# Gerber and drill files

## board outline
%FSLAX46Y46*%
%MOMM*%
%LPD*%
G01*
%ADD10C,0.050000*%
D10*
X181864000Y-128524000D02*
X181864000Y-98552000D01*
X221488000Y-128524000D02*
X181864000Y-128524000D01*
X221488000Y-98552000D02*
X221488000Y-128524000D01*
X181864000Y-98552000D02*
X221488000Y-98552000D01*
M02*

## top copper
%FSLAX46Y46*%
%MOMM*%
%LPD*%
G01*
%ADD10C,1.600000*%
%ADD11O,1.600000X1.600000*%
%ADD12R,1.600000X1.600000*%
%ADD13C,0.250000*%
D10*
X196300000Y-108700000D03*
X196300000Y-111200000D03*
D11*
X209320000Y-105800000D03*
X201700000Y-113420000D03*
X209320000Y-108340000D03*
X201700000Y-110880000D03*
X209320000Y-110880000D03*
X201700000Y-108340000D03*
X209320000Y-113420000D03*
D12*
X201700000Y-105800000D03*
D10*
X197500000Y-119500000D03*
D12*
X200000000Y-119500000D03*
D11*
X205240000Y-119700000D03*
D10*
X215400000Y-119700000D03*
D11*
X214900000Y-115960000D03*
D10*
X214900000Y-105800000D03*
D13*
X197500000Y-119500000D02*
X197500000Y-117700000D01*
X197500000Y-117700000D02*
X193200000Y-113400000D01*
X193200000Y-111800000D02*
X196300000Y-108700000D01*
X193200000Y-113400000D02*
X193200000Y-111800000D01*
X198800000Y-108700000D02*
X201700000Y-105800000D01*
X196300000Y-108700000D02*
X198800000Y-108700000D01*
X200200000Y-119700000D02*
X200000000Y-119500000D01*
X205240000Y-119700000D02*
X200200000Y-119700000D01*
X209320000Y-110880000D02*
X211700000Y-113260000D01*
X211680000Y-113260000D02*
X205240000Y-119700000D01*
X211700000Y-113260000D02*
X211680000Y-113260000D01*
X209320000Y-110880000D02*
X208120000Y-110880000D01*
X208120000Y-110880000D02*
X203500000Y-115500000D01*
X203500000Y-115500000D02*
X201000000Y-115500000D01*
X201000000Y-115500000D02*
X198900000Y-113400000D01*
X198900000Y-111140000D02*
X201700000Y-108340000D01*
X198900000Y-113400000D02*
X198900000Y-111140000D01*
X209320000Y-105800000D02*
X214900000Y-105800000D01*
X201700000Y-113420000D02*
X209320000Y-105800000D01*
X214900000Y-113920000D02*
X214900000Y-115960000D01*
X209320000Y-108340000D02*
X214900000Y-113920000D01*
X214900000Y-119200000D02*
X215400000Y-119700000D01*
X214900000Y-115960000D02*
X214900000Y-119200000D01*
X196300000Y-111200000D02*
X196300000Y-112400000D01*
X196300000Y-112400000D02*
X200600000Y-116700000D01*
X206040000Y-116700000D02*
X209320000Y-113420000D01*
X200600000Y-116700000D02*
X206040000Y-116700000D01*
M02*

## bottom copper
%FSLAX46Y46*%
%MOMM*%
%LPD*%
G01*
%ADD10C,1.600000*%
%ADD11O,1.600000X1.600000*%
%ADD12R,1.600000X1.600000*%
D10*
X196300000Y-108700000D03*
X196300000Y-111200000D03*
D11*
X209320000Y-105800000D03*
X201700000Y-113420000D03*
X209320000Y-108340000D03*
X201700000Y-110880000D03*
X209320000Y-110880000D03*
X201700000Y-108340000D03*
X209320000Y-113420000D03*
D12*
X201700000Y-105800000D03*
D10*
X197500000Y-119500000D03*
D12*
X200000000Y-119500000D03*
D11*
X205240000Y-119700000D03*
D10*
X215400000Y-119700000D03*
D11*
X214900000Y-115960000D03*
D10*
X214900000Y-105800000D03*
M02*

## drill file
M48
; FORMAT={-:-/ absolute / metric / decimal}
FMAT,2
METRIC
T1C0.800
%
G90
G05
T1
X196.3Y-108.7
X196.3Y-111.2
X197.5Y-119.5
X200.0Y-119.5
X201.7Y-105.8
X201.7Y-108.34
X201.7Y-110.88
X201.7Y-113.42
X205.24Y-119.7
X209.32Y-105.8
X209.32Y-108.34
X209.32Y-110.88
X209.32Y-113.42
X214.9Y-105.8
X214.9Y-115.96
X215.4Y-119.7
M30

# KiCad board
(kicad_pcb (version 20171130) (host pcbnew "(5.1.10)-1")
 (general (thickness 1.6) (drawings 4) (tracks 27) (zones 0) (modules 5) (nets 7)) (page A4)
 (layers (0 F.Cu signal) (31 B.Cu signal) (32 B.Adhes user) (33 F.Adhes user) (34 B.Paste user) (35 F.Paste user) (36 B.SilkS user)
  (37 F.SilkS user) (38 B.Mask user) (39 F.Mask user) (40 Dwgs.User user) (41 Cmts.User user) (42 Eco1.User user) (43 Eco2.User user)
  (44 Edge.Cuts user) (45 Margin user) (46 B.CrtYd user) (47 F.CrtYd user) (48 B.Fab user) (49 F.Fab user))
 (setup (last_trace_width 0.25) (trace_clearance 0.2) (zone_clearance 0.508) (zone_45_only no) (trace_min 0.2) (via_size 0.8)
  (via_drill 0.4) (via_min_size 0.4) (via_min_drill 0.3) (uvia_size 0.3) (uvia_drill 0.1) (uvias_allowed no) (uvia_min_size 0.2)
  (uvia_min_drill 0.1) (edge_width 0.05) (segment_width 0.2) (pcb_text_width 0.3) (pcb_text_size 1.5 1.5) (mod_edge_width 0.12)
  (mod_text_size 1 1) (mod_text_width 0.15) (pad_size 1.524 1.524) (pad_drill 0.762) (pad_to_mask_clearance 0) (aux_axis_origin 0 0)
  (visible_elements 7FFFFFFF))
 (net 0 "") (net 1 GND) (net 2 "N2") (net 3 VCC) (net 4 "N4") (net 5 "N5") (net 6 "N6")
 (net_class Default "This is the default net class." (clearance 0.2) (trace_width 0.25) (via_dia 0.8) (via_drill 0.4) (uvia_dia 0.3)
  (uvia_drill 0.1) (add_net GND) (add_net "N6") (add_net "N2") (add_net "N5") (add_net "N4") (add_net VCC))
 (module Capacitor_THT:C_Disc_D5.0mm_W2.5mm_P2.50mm (layer F.Cu) (at 196.3 111.2 90)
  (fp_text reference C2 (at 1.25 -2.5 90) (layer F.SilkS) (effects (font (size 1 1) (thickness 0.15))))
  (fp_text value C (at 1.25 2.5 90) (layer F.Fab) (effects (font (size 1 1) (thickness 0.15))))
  (pad 2 thru_hole circle (at 2.5 0 90) (size 1.6 1.6) (drill 0.8) (layers *.Cu *.Mask) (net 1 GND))
  (pad 1 thru_hole circle (at 0 0 90) (size 1.6 1.6) (drill 0.8) (layers *.Cu *.Mask) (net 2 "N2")))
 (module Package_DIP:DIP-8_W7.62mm (layer F.Cu) (at 201.7 105.8)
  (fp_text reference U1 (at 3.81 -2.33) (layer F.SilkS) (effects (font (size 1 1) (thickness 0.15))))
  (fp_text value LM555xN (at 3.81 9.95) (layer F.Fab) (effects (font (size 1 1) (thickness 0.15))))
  (pad 8 thru_hole oval (at 7.62 0) (size 1.6 1.6) (drill 0.8) (layers *.Cu *.Mask) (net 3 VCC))
  (pad 4 thru_hole oval (at 0 7.62) (size 1.6 1.6) (drill 0.8) (layers *.Cu *.Mask) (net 3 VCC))
  (pad 7 thru_hole oval (at 7.62 2.54) (size 1.6 1.6) (drill 0.8) (layers *.Cu *.Mask) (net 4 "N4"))
  (pad 3 thru_hole oval (at 0 5.08) (size 1.6 1.6) (drill 0.8) (layers *.Cu *.Mask) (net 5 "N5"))
  (pad 6 thru_hole oval (at 7.62 5.08) (size 1.6 1.6) (drill 0.8) (layers *.Cu *.Mask) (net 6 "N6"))
  (pad 2 thru_hole oval (at 0 2.54) (size 1.6 1.6) (drill 0.8) (layers *.Cu *.Mask) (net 6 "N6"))
  (pad 5 thru_hole oval (at 7.62 7.62) (size 1.6 1.6) (drill 0.8) (layers *.Cu *.Mask) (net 2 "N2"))
  (pad 1 thru_hole rect (at 0 0) (size 1.6 1.6) (drill 0.8) (layers *.Cu *.Mask) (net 1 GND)))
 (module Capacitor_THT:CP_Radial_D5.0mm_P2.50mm (layer F.Cu) (at 200 119.5 180)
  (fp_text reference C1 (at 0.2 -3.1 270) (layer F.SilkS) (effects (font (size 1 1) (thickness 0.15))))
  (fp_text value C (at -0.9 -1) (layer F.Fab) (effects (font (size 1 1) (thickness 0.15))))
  (pad 2 thru_hole circle (at 2.5 0 180) (size 1.6 1.6) (drill 0.8) (layers *.Cu *.Mask) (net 1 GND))
  (pad 1 thru_hole rect (at 0 0 180) (size 1.6 1.6) (drill 0.8) (layers *.Cu *.Mask) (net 6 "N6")))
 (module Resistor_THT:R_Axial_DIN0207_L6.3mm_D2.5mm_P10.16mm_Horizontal (layer F.Cu) (at 215.4 119.7 180)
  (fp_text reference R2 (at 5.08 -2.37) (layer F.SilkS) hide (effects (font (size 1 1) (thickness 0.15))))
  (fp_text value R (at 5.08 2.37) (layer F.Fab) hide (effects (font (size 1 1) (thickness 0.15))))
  (pad 2 thru_hole oval (at 10.16 0 180) (size 1.6 1.6) (drill 0.8) (layers *.Cu *.Mask) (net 6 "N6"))
  (pad 1 thru_hole circle (at 0 0 180) (size 1.6 1.6) (drill 0.8) (layers *.Cu *.Mask) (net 4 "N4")))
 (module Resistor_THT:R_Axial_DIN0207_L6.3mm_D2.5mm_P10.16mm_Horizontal (layer F.Cu) (at 214.9 105.8 270)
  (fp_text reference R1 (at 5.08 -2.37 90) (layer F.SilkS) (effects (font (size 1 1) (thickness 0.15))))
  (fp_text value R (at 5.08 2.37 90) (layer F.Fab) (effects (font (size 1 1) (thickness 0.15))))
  (pad 2 thru_hole oval (at 10.16 0 270) (size 1.6 1.6) (drill 0.8) (layers *.Cu *.Mask) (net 4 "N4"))
  (pad 1 thru_hole circle (at 0 0 270) (size 1.6 1.6) (drill 0.8) (layers *.Cu *.Mask) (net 3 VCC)))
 (gr_line (start 181.864 128.524) (end 181.864 98.552) (layer Edge.Cuts) (width 0.05))
 (gr_line (start 221.488 128.524) (end 181.864 128.524) (layer Edge.Cuts) (width 0.05))
 (gr_line (start 221.488 98.552) (end 221.488 128.524) (layer Edge.Cuts) (width 0.05))
 (gr_line (start 181.864 98.552) (end 221.488 98.552) (layer Edge.Cuts) (width 0.05))
 (segment (start 197.5 119.5) (end 197.5 117.7) (width 0.25) (layer F.Cu) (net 1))
 (segment (start 197.5 117.7) (end 193.2 113.4) (width 0.25) (layer F.Cu) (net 1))
 (segment (start 193.2 111.8) (end 196.3 108.7) (width 0.25) (layer F.Cu) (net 1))
 (segment (start 193.2 113.4) (end 193.2 111.8) (width 0.25) (layer F.Cu) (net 1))
 (segment (start 198.8 108.7) (end 201.7 105.8) (width 0.25) (layer F.Cu) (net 1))
 (segment (start 196.3 108.7) (end 198.8 108.7) (width 0.25) (layer F.Cu) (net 1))
 (segment (start 200.2 119.7) (end 200 119.5) (width 0.25) (layer F.Cu) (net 6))
 (segment (start 205.24 119.7) (end 200.2 119.7) (width 0.25) (layer F.Cu) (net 6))
 (segment (start 209.32 110.88) (end 211.7 113.26) (width 0.25) (layer F.Cu) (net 6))
 (segment (start 211.68 113.26) (end 205.24 119.7) (width 0.25) (layer F.Cu) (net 6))
 (segment (start 211.7 113.26) (end 211.68 113.26) (width 0.25) (layer F.Cu) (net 6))
 (segment (start 209.32 110.88) (end 208.12 110.88) (width 0.25) (layer F.Cu) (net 6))
 (segment (start 208.12 110.88) (end 203.5 115.5) (width 0.25) (layer F.Cu) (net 6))
 (segment (start 203.5 115.5) (end 201 115.5) (width 0.25) (layer F.Cu) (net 6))
 (segment (start 201 115.5) (end 198.9 113.4) (width 0.25) (layer F.Cu) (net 6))
 (segment (start 198.9 111.14) (end 201.7 108.34) (width 0.25) (layer F.Cu) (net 6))
 (segment (start 198.9 113.4) (end 198.9 111.14) (width 0.25) (layer F.Cu) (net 6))
 (segment (start 209.32 105.8) (end 214.9 105.8) (width 0.25) (layer F.Cu) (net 3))
 (segment (start 201.7 113.42) (end 209.32 105.8) (width 0.25) (layer F.Cu) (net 3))
 (segment (start 214.9 113.92) (end 214.9 115.96) (width 0.25) (layer F.Cu) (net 4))
 (segment (start 209.32 108.34) (end 214.9 113.92) (width 0.25) (layer F.Cu) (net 4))
 (segment (start 214.9 119.2) (end 215.4 119.7) (width 0.25) (layer F.Cu) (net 4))
 (segment (start 214.9 115.96) (end 214.9 119.2) (width 0.25) (layer F.Cu) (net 4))
 (segment (start 196.3 111.2) (end 196.3 112.4) (width 0.25) (layer F.Cu) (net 2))
 (segment (start 196.3 112.4) (end 200.6 116.7) (width 0.25) (layer F.Cu) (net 2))
 (segment (start 206.04 116.7) (end 209.32 113.42) (width 0.25) (layer F.Cu) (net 2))
 (segment (start 200.6 116.7) (end 206.04 116.7) (width 0.25) (layer F.Cu) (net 2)))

